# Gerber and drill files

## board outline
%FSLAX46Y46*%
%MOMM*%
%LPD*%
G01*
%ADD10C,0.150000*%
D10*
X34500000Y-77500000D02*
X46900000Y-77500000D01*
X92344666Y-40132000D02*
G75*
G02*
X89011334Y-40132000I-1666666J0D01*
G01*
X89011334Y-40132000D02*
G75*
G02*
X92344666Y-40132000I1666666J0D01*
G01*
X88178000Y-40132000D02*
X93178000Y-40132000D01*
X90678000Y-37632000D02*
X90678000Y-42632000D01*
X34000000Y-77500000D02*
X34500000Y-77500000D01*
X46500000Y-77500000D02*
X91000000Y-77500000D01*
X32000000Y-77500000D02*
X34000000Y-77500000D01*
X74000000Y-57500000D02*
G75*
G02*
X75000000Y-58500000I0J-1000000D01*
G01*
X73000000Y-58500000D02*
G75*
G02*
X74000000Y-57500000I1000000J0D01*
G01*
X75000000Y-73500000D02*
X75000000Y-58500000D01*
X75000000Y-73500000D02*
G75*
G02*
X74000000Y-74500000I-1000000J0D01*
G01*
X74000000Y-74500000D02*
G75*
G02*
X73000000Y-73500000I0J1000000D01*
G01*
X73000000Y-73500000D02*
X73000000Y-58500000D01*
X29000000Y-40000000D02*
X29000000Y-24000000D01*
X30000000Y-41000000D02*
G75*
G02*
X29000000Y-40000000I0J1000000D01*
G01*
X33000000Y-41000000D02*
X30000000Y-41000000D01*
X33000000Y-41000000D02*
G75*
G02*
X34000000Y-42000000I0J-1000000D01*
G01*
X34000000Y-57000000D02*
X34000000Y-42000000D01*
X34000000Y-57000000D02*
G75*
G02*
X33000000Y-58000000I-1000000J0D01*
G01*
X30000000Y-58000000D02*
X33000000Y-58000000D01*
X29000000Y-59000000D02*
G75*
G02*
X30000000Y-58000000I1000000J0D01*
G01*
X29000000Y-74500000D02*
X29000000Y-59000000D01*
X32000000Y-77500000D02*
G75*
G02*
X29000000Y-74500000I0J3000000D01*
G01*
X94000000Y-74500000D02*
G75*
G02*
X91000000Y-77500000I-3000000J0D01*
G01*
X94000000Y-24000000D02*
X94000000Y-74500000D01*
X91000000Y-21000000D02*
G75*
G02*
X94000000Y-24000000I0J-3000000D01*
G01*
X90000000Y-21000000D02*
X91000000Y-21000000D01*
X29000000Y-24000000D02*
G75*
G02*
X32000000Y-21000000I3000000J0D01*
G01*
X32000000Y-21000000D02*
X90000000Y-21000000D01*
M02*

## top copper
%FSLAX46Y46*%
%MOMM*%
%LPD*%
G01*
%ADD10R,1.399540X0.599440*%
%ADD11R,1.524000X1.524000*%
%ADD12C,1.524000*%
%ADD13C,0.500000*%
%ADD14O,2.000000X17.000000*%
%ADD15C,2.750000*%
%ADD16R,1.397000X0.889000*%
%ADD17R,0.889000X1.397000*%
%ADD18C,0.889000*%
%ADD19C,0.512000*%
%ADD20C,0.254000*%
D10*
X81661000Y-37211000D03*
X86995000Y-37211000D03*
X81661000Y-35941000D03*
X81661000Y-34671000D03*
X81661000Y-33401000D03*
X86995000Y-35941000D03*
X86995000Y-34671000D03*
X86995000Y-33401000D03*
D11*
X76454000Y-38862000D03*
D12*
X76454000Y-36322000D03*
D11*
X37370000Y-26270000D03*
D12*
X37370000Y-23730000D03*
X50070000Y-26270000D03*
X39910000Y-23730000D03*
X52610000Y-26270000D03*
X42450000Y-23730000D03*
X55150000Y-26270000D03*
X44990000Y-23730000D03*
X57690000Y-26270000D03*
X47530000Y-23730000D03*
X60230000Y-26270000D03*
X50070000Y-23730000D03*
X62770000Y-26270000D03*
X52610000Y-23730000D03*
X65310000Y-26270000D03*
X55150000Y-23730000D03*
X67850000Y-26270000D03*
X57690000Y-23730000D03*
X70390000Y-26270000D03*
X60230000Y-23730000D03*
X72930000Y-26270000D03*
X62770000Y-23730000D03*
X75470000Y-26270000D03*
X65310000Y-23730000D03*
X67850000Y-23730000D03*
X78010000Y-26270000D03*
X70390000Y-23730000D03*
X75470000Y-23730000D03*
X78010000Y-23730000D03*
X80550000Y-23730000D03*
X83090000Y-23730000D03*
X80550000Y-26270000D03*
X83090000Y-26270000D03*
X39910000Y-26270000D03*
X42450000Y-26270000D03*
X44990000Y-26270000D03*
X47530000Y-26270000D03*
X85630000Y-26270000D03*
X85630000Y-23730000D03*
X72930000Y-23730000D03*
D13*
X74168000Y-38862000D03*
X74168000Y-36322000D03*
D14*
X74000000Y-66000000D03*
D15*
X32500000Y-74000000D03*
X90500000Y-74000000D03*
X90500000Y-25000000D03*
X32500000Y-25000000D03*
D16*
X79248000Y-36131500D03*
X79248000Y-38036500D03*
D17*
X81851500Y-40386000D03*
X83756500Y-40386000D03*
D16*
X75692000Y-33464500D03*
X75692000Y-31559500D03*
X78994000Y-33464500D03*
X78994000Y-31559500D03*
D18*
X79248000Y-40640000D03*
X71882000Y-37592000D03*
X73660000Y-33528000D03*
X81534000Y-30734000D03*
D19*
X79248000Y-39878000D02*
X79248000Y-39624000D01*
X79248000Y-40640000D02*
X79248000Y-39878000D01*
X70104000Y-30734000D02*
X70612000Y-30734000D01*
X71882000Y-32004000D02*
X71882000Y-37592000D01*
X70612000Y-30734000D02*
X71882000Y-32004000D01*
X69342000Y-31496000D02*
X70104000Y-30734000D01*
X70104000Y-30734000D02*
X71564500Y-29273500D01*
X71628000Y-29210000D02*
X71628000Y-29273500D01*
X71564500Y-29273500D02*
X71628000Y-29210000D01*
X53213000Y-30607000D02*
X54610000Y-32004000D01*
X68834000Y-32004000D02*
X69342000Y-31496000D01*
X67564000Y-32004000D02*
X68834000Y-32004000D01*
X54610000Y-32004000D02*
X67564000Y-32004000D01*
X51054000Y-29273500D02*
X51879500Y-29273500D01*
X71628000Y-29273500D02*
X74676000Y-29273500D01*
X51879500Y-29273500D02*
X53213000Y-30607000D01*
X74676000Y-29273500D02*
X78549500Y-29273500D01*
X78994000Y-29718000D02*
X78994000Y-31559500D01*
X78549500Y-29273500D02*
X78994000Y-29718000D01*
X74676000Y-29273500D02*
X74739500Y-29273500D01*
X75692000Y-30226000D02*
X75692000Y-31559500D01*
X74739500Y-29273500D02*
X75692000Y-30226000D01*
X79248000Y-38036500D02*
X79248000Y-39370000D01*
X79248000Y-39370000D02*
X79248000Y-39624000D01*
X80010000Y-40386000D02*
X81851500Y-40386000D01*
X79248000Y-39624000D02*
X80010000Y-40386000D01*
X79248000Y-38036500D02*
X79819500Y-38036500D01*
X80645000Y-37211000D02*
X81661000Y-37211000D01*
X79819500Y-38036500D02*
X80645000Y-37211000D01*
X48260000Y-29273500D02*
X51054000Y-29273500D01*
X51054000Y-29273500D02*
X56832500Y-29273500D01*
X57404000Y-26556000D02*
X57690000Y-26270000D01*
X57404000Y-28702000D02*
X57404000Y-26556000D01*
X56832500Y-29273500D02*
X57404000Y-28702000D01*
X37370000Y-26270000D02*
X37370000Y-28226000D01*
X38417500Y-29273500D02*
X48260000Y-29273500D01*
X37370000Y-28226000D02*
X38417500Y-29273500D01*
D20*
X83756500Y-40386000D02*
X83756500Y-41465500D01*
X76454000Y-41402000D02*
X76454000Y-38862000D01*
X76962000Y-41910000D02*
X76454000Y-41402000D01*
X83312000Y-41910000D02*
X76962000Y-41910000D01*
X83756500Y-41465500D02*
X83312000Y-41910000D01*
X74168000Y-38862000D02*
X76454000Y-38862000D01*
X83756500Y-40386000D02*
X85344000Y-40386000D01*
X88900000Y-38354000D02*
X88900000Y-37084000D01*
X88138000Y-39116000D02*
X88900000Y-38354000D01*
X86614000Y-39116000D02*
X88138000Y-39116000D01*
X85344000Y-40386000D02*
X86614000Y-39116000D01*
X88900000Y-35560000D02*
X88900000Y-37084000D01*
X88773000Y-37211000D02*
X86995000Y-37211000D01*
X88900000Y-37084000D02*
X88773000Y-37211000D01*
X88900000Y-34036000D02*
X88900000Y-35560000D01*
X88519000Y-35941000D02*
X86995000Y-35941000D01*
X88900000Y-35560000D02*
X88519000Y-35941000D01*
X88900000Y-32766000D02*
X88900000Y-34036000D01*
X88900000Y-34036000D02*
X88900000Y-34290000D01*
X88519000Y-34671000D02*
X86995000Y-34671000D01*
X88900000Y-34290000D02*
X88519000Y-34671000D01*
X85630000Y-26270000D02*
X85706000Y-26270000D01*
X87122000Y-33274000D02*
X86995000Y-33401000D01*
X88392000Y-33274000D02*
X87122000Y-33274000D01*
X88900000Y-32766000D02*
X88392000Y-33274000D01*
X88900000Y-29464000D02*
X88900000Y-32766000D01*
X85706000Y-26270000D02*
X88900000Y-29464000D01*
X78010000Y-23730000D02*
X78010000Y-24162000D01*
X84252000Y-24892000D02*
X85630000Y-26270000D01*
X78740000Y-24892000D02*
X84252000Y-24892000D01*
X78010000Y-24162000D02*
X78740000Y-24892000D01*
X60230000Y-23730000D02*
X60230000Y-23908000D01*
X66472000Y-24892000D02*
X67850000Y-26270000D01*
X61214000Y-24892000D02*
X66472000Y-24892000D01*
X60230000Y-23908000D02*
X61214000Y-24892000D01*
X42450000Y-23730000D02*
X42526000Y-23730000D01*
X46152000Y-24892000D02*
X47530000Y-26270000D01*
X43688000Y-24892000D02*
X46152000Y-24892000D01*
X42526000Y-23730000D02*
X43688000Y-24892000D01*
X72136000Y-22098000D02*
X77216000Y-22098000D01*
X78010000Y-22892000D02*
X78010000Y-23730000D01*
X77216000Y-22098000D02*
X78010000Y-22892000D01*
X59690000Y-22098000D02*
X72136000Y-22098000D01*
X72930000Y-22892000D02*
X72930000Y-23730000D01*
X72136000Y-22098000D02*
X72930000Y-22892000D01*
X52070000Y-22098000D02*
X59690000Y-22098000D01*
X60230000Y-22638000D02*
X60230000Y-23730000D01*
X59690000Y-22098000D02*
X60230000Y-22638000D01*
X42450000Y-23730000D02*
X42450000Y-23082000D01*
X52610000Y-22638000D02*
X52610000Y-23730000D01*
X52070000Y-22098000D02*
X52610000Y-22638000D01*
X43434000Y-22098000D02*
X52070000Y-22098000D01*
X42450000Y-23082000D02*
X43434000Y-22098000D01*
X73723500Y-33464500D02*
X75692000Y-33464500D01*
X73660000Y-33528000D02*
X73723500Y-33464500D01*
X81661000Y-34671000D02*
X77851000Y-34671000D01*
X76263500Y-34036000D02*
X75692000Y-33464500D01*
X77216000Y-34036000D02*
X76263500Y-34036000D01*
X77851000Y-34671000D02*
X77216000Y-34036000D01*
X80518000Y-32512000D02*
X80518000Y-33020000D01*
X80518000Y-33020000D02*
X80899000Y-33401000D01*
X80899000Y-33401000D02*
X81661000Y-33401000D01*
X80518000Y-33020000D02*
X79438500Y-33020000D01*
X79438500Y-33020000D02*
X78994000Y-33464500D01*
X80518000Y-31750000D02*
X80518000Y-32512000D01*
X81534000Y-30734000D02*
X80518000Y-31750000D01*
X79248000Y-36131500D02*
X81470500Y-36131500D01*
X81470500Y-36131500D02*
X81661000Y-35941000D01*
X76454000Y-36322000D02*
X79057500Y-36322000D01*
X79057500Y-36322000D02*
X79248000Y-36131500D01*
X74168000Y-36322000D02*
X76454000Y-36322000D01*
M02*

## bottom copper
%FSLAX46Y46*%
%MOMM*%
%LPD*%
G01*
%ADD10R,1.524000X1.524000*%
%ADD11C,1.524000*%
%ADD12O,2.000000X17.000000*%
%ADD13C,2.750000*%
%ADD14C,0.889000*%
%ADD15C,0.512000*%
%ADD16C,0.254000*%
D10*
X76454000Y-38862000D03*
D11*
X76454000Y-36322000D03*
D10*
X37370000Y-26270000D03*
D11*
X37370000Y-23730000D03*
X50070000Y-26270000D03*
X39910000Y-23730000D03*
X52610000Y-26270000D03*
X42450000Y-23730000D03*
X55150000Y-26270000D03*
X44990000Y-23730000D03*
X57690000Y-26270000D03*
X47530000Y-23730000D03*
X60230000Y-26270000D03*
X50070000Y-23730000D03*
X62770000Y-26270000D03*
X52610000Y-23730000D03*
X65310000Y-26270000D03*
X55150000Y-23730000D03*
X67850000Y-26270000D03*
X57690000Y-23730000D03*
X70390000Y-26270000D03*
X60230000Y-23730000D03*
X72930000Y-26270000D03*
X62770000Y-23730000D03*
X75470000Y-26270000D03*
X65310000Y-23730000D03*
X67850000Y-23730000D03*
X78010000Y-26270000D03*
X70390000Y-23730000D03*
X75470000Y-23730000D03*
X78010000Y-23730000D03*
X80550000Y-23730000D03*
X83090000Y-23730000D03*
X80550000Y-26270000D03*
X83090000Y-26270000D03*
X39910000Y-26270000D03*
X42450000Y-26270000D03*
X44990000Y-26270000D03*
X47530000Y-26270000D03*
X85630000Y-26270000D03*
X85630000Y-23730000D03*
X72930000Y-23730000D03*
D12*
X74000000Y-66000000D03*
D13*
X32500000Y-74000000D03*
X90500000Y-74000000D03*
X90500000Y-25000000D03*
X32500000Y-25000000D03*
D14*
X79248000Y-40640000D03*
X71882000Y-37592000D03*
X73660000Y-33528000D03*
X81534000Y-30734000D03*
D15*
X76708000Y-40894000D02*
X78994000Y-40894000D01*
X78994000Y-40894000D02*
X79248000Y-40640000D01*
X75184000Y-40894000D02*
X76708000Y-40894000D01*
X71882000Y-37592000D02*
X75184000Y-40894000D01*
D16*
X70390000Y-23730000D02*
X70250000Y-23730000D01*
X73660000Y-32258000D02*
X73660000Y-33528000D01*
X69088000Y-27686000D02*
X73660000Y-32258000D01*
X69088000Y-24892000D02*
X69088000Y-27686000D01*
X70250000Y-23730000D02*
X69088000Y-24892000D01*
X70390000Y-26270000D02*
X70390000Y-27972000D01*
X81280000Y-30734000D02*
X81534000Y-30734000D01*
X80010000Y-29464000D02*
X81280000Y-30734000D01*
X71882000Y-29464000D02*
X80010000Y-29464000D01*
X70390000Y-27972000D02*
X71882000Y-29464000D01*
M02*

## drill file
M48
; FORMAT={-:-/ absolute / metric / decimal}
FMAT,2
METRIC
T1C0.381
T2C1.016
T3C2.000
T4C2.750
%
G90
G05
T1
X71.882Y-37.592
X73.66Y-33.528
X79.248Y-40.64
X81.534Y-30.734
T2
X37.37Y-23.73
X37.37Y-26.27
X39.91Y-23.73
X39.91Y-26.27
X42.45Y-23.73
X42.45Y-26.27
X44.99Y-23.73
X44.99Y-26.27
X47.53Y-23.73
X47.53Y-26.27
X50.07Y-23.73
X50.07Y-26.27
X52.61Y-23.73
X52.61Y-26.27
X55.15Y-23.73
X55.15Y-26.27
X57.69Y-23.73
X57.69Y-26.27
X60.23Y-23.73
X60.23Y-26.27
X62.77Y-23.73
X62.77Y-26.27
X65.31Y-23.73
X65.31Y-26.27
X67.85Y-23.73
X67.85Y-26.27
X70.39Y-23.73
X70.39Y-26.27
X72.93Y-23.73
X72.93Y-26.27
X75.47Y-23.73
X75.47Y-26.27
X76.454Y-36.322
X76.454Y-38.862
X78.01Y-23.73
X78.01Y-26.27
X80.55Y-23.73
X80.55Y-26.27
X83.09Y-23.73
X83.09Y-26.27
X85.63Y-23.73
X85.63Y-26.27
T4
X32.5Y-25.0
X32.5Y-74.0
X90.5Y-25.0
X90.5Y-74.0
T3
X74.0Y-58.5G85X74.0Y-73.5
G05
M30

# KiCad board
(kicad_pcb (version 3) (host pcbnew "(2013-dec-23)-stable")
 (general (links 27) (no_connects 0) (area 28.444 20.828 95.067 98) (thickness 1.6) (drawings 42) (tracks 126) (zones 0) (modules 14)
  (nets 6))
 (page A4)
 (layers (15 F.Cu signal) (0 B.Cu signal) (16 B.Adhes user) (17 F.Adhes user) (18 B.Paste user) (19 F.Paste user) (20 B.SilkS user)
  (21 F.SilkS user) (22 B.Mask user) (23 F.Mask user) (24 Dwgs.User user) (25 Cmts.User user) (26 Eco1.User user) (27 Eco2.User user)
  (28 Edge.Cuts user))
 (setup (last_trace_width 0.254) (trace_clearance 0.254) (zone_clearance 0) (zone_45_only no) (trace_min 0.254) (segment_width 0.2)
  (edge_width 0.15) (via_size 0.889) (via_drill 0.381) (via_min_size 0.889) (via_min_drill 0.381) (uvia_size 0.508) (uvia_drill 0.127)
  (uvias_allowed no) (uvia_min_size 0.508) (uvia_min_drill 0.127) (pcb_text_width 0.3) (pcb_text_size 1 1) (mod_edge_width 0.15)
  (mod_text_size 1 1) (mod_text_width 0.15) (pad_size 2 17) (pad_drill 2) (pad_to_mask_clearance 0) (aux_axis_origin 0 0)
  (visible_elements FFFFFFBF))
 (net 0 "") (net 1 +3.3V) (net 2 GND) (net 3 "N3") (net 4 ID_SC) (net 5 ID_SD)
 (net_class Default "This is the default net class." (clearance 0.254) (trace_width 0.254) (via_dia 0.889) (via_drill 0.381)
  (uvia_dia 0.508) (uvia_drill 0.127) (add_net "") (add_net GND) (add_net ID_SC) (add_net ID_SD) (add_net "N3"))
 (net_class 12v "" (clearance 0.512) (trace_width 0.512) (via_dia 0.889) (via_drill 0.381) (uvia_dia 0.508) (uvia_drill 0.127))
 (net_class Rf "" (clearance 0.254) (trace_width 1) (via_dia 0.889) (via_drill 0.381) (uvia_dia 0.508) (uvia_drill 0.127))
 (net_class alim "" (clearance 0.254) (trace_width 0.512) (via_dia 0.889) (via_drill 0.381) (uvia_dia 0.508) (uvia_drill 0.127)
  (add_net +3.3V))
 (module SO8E (layer F.Cu) (at 84.328 35.306 90)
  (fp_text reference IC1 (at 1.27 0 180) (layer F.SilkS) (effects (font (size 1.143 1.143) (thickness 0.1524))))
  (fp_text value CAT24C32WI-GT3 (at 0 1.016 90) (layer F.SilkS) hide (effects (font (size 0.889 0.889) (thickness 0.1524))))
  (pad 8 smd rect (at -1.905 -2.667 90) (size 0.59944 1.39954) (layers F.Cu F.Paste F.Mask) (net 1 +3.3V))
  (pad 1 smd rect (at -1.905 2.667 90) (size 0.59944 1.39954) (layers F.Cu F.Paste F.Mask) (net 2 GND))
  (pad 7 smd rect (at -0.635 -2.667 90) (size 0.59944 1.39954) (layers F.Cu F.Paste F.Mask) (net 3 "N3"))
  (pad 6 smd rect (at 0.635 -2.667 90) (size 0.59944 1.39954) (layers F.Cu F.Paste F.Mask) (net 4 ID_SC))
  (pad 5 smd rect (at 1.905 -2.667 90) (size 0.59944 1.39954) (layers F.Cu F.Paste F.Mask) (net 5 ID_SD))
  (pad 2 smd rect (at -0.635 2.667 90) (size 0.59944 1.39954) (layers F.Cu F.Paste F.Mask) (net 2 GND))
  (pad 3 smd rect (at 0.635 2.667 90) (size 0.59944 1.39954) (layers F.Cu F.Paste F.Mask) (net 2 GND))
  (pad 4 smd rect (at 1.905 2.667 90) (size 0.59944 1.39954) (layers F.Cu F.Paste F.Mask) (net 2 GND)))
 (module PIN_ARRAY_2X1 (layer F.Cu) (at 76.454 37.592 90)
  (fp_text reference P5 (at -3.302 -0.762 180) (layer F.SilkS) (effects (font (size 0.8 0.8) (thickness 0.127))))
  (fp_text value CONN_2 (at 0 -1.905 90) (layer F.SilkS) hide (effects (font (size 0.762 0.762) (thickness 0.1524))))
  (pad 1 thru_hole rect (at -1.27 0 90) (size 1.524 1.524) (drill 1.016) (layers *.Cu *.Mask F.SilkS) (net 2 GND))
  (pad 2 thru_hole circle (at 1.27 0 90) (size 1.524 1.524) (drill 1.016) (layers *.Cu *.Mask F.SilkS) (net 3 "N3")))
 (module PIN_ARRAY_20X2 (layer F.Cu) (at 61.5 25)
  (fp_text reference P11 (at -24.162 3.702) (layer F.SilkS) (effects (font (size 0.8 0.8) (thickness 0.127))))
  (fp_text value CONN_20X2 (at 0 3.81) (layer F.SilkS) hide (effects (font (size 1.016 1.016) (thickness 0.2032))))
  (pad 1 thru_hole rect (at -24.13 1.27) (size 1.524 1.524) (drill 1.016) (layers *.Cu *.Mask F.SilkS) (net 1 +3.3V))
  (pad 2 thru_hole circle (at -24.13 -1.27) (size 1.524 1.524) (drill 1.016) (layers *.Cu *.Mask F.SilkS))
  (pad 11 thru_hole circle (at -11.43 1.27) (size 1.524 1.524) (drill 1.016) (layers *.Cu *.Mask F.SilkS))
  (pad 4 thru_hole circle (at -21.59 -1.27) (size 1.524 1.524) (drill 1.016) (layers *.Cu *.Mask F.SilkS))
  (pad 13 thru_hole circle (at -8.89 1.27) (size 1.524 1.524) (drill 1.016) (layers *.Cu *.Mask F.SilkS))
  (pad 6 thru_hole circle (at -19.05 -1.27) (size 1.524 1.524) (drill 1.016) (layers *.Cu *.Mask F.SilkS) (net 2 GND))
  (pad 15 thru_hole circle (at -6.35 1.27) (size 1.524 1.524) (drill 1.016) (layers *.Cu *.Mask F.SilkS))
  (pad 8 thru_hole circle (at -16.51 -1.27) (size 1.524 1.524) (drill 1.016) (layers *.Cu *.Mask F.SilkS))
  (pad 17 thru_hole circle (at -3.81 1.27) (size 1.524 1.524) (drill 1.016) (layers *.Cu *.Mask F.SilkS) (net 1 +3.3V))
  (pad 10 thru_hole circle (at -13.97 -1.27) (size 1.524 1.524) (drill 1.016) (layers *.Cu *.Mask F.SilkS))
  (pad 19 thru_hole circle (at -1.27 1.27) (size 1.524 1.524) (drill 1.016) (layers *.Cu *.Mask F.SilkS))
  (pad 12 thru_hole circle (at -11.43 -1.27) (size 1.524 1.524) (drill 1.016) (layers *.Cu *.Mask F.SilkS))
  (pad 21 thru_hole circle (at 1.27 1.27) (size 1.524 1.524) (drill 1.016) (layers *.Cu *.Mask F.SilkS))
  (pad 14 thru_hole circle (at -8.89 -1.27) (size 1.524 1.524) (drill 1.016) (layers *.Cu *.Mask F.SilkS) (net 2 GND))
  (pad 23 thru_hole circle (at 3.81 1.27) (size 1.524 1.524) (drill 1.016) (layers *.Cu *.Mask F.SilkS))
  (pad 16 thru_hole circle (at -6.35 -1.27) (size 1.524 1.524) (drill 1.016) (layers *.Cu *.Mask F.SilkS))
  (pad 25 thru_hole circle (at 6.35 1.27) (size 1.524 1.524) (drill 1.016) (layers *.Cu *.Mask F.SilkS) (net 2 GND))
  (pad 18 thru_hole circle (at -3.81 -1.27) (size 1.524 1.524) (drill 1.016) (layers *.Cu *.Mask F.SilkS))
  (pad 27 thru_hole circle (at 8.89 1.27) (size 1.524 1.524) (drill 1.016) (layers *.Cu *.Mask F.SilkS) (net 5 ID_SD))
  (pad 20 thru_hole circle (at -1.27 -1.27) (size 1.524 1.524) (drill 1.016) (layers *.Cu *.Mask F.SilkS) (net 2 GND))
  (pad 29 thru_hole circle (at 11.43 1.27) (size 1.524 1.524) (drill 1.016) (layers *.Cu *.Mask F.SilkS))
  (pad 22 thru_hole circle (at 1.27 -1.27) (size 1.524 1.524) (drill 1.016) (layers *.Cu *.Mask F.SilkS))
  (pad 31 thru_hole circle (at 13.97 1.27) (size 1.524 1.524) (drill 1.016) (layers *.Cu *.Mask F.SilkS))
  (pad 24 thru_hole circle (at 3.81 -1.27) (size 1.524 1.524) (drill 1.016) (layers *.Cu *.Mask F.SilkS))
  (pad 26 thru_hole circle (at 6.35 -1.27) (size 1.524 1.524) (drill 1.016) (layers *.Cu *.Mask F.SilkS))
  (pad 33 thru_hole circle (at 16.51 1.27) (size 1.524 1.524) (drill 1.016) (layers *.Cu *.Mask F.SilkS))
  (pad 28 thru_hole circle (at 8.89 -1.27) (size 1.524 1.524) (drill 1.016) (layers *.Cu *.Mask F.SilkS) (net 4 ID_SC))
  (pad 32 thru_hole circle (at 13.97 -1.27) (size 1.524 1.524) (drill 1.016) (layers *.Cu *.Mask F.SilkS))
  (pad 34 thru_hole circle (at 16.51 -1.27) (size 1.524 1.524) (drill 1.016) (layers *.Cu *.Mask F.SilkS) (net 2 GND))
  (pad 36 thru_hole circle (at 19.05 -1.27) (size 1.524 1.524) (drill 1.016) (layers *.Cu *.Mask F.SilkS))
  (pad 38 thru_hole circle (at 21.59 -1.27) (size 1.524 1.524) (drill 1.016) (layers *.Cu *.Mask F.SilkS))
  (pad 35 thru_hole circle (at 19.05 1.27) (size 1.524 1.524) (drill 1.016) (layers *.Cu *.Mask F.SilkS))
  (pad 37 thru_hole circle (at 21.59 1.27) (size 1.524 1.524) (drill 1.016) (layers *.Cu *.Mask F.SilkS))
  (pad 3 thru_hole circle (at -21.59 1.27) (size 1.524 1.524) (drill 1.016) (layers *.Cu *.Mask F.SilkS))
  (pad 5 thru_hole circle (at -19.05 1.27) (size 1.524 1.524) (drill 1.016) (layers *.Cu *.Mask F.SilkS))
  (pad 7 thru_hole circle (at -16.51 1.27) (size 1.524 1.524) (drill 1.016) (layers *.Cu *.Mask F.SilkS))
  (pad 9 thru_hole circle (at -13.97 1.27) (size 1.524 1.524) (drill 1.016) (layers *.Cu *.Mask F.SilkS) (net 2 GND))
  (pad 39 thru_hole circle (at 24.13 1.27) (size 1.524 1.524) (drill 1.016) (layers *.Cu *.Mask F.SilkS) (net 2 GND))
  (pad 40 thru_hole circle (at 24.13 -1.27) (size 1.524 1.524) (drill 1.016) (layers *.Cu *.Mask F.SilkS))
  (pad 30 thru_hole circle (at 11.43 -1.27) (size 1.524 1.524) (drill 1.016) (layers *.Cu *.Mask F.SilkS) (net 2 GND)))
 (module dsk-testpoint (layer F.Cu) (at 74.168 38.862)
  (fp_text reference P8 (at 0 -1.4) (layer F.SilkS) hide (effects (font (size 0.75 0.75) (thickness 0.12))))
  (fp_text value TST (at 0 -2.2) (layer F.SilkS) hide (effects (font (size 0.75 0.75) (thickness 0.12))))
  (pad 1 smd circle (at 0 0) (size 0.5 0.5) (layers F.Cu F.Paste F.Mask) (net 2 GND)))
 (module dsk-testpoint (layer F.Cu) (at 74.168 36.322)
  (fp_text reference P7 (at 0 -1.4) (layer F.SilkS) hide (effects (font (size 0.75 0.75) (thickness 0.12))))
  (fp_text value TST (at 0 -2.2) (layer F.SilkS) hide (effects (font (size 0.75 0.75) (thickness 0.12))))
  (pad 1 smd circle (at 0 0) (size 0.5 0.5) (layers F.Cu F.Paste F.Mask) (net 3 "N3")))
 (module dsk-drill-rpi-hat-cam (layer F.Cu) (at 74 66)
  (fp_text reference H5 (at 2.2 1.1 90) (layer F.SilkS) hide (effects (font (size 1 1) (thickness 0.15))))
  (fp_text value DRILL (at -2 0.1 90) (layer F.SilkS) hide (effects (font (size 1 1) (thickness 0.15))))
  (pad 1 thru_hole oval (at 0 0) (size 2 17) (drill oval 2 17) (layers *.Cu F.SilkS) (solder_mask_margin 0.254) (clearance 0.254)))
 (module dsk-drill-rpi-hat (layer F.Cu) (at 32.5 74)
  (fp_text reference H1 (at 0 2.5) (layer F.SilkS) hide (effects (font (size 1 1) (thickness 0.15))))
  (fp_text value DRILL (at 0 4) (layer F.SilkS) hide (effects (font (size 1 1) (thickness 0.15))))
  (pad 1 thru_hole circle (at 0 0) (size 2.75 2.75) (drill 2.75) (layers *.Cu) (solder_mask_margin 1.725) (clearance 1.725) (zone_connect 0)))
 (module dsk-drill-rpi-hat (layer F.Cu) (at 90.5 74)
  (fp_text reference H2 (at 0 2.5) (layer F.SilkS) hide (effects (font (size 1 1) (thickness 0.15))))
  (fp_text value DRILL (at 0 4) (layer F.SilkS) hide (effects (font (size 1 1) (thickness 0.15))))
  (pad 1 thru_hole circle (at 0 0) (size 2.75 2.75) (drill 2.75) (layers *.Cu) (solder_mask_margin 1.725) (clearance 1.725) (zone_connect 0)))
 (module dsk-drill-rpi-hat (layer F.Cu) (at 90.5 25)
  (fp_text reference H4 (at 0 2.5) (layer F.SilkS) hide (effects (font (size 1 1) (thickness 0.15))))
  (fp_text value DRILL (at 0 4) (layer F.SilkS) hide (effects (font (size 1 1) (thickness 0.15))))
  (pad 1 thru_hole circle (at 0 0) (size 2.75 2.75) (drill 2.75) (layers *.Cu) (solder_mask_margin 1.725) (clearance 1.725) (zone_connect 0)))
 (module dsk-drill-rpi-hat (layer F.Cu) (at 32.5 25)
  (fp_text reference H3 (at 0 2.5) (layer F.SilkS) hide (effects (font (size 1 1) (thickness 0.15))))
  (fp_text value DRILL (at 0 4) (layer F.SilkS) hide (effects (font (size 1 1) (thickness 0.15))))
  (pad 1 thru_hole circle (at 0 0) (size 2.75 2.75) (drill 2.75) (layers *.Cu) (solder_mask_margin 1.725) (clearance 1.725) (zone_connect 0)))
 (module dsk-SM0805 (layer F.Cu) (at 79.248 37.084 270)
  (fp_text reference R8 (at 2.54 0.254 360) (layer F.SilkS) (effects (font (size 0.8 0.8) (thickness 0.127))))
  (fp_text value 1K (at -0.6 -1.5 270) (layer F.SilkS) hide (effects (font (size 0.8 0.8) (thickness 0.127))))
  (pad 1 smd rect (at -0.9525 0 270) (size 0.889 1.397) (layers F.Cu F.Paste F.Mask) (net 3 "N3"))
  (pad 2 smd rect (at 0.9525 0 270) (size 0.889 1.397) (layers F.Cu F.Paste F.Mask) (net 1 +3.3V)))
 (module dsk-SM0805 (layer F.Cu) (at 82.804 40.386)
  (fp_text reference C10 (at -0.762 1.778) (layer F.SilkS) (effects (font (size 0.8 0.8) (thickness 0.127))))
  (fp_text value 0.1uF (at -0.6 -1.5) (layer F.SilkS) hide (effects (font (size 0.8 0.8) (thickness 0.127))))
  (pad 1 smd rect (at -0.9525 0) (size 0.889 1.397) (layers F.Cu F.Paste F.Mask) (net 1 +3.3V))
  (pad 2 smd rect (at 0.9525 0) (size 0.889 1.397) (layers F.Cu F.Paste F.Mask) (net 2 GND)))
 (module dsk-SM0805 (layer F.Cu) (at 75.692 32.512 90)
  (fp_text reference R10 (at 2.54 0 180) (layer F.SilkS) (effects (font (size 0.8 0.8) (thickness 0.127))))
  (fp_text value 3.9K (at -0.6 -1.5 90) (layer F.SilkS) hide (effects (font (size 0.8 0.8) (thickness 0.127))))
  (pad 1 smd rect (at -0.9525 0 90) (size 0.889 1.397) (layers F.Cu F.Paste F.Mask) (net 4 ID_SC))
  (pad 2 smd rect (at 0.9525 0 90) (size 0.889 1.397) (layers F.Cu F.Paste F.Mask) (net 1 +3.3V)))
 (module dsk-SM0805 (layer F.Cu) (at 78.994 32.512 90)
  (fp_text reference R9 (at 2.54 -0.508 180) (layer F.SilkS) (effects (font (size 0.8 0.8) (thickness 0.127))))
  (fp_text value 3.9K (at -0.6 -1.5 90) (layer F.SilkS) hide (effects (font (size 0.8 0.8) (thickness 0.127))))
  (pad 1 smd rect (at -0.9525 0 90) (size 0.889 1.397) (layers F.Cu F.Paste F.Mask) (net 5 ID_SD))
  (pad 2 smd rect (at 0.9525 0 90) (size 0.889 1.397) (layers F.Cu F.Paste F.Mask) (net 1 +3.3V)))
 (gr_line (start 34.5 77.5) (end 46.9 77.5) (angle 90) (layer Edge.Cuts) (width 0.15))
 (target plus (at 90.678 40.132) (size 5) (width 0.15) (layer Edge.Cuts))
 (gr_line (start 34 77.5) (end 34.5 77.5) (angle 90) (layer Edge.Cuts) (width 0.15))
 (gr_line (start 46.5 77.5) (end 91 77.5) (angle 90) (layer Edge.Cuts) (width 0.15))
 (gr_line (start 32 77.5) (end 34 77.5) (angle 90) (layer Edge.Cuts) (width 0.15))
 (gr_arc (start 74 58.5) (end 74 57.5) (angle 90) (layer Edge.Cuts) (width 0.15))
 (gr_arc (start 74 58.5) (end 73 58.5) (angle 90) (layer Edge.Cuts) (width 0.15))
 (gr_line (start 75 73.5) (end 75 58.5) (angle 90) (layer Edge.Cuts) (width 0.15))
 (gr_arc (start 74 73.5) (end 75 73.5) (angle 90) (layer Edge.Cuts) (width 0.15))
 (gr_arc (start 74 73.5) (end 74 74.5) (angle 90) (layer Edge.Cuts) (width 0.15))
 (gr_line (start 73 73.5) (end 73 58.5) (angle 90) (layer Edge.Cuts) (width 0.15))
 (gr_line (start 29 40) (end 29 24) (angle 90) (layer Edge.Cuts) (width 0.15))
 (gr_arc (start 30 40) (end 30 41) (angle 90) (layer Edge.Cuts) (width 0.15))
 (gr_line (start 33 41) (end 30 41) (angle 90) (layer Edge.Cuts) (width 0.15))
 (gr_arc (start 33 42) (end 33 41) (angle 90) (layer Edge.Cuts) (width 0.15))
 (gr_line (start 34 57) (end 34 42) (angle 90) (layer Edge.Cuts) (width 0.15))
 (gr_arc (start 33 57) (end 34 57) (angle 90) (layer Edge.Cuts) (width 0.15))
 (gr_line (start 30 58) (end 33 58) (angle 90) (layer Edge.Cuts) (width 0.15))
 (gr_arc (start 30 59) (end 29 59) (angle 90) (layer Edge.Cuts) (width 0.15))
 (gr_line (start 29 74.5) (end 29 59) (angle 90) (layer Edge.Cuts) (width 0.15))
 (gr_arc (start 32 74.5) (end 32 77.5) (angle 90) (layer Edge.Cuts) (width 0.15))
 (gr_arc (start 91 74.5) (end 94 74.5) (angle 90) (layer Edge.Cuts) (width 0.15))
 (gr_line (start 94 24) (end 94 74.5) (angle 90) (layer Edge.Cuts) (width 0.15))
 (gr_arc (start 91 24) (end 91 21) (angle 90) (layer Edge.Cuts) (width 0.15))
 (gr_line (start 90 21) (end 91 21) (angle 90) (layer Edge.Cuts) (width 0.15))
 (gr_arc (start 32 24) (end 29 24) (angle 90) (layer Edge.Cuts) (width 0.15))
 (gr_line (start 32 21) (end 90 21) (angle 90) (layer Edge.Cuts) (width 0.15))
 (segment (start 76.708 40.894) (end 78.994 40.894) (width 0.512) (layer B.Cu) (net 1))
 (segment (start 79.248 39.878) (end 79.248 39.624) (width 0.512) (layer F.Cu) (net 1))
 (segment (start 79.248 40.64) (end 79.248 39.878) (width 0.512) (layer F.Cu) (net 1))
 (via (at 79.248 40.64) (size 0.889) (layers F.Cu B.Cu) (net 1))
 (segment (start 78.994 40.894) (end 79.248 40.64) (width 0.512) (layer B.Cu) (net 1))
 (segment (start 70.104 30.734) (end 70.612 30.734) (width 0.512) (layer F.Cu) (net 1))
 (segment (start 75.184 40.894) (end 76.708 40.894) (width 0.512) (layer B.Cu) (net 1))
 (segment (start 71.882 37.592) (end 75.184 40.894) (width 0.512) (layer B.Cu) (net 1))
 (via (at 71.882 37.592) (size 0.889) (layers F.Cu B.Cu) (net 1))
 (segment (start 71.882 32.004) (end 71.882 37.592) (width 0.512) (layer F.Cu) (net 1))
 (segment (start 70.612 30.734) (end 71.882 32.004) (width 0.512) (layer F.Cu) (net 1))
 (segment (start 69.342 31.496) (end 70.104 30.734) (width 0.512) (layer F.Cu) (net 1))
 (segment (start 70.104 30.734) (end 71.5645 29.2735) (width 0.512) (layer F.Cu) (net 1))
 (segment (start 71.628 29.21) (end 71.628 29.2735) (width 0.512) (layer F.Cu) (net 1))
 (segment (start 71.5645 29.2735) (end 71.628 29.21) (width 0.512) (layer F.Cu) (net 1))
 (segment (start 53.213 30.607) (end 54.61 32.004) (width 0.512) (layer F.Cu) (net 1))
 (segment (start 68.834 32.004) (end 69.342 31.496) (width 0.512) (layer F.Cu) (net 1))
 (segment (start 67.564 32.004) (end 68.834 32.004) (width 0.512) (layer F.Cu) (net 1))
 (segment (start 54.61 32.004) (end 67.564 32.004) (width 0.512) (layer F.Cu) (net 1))
 (segment (start 51.054 29.2735) (end 51.8795 29.2735) (width 0.512) (layer F.Cu) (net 1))
 (segment (start 71.628 29.2735) (end 74.676 29.2735) (width 0.512) (layer F.Cu) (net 1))
 (segment (start 51.8795 29.2735) (end 53.213 30.607) (width 0.512) (layer F.Cu) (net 1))
 (segment (start 74.676 29.2735) (end 78.5495 29.2735) (width 0.512) (layer F.Cu) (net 1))
 (segment (start 78.994 29.718) (end 78.994 31.5595) (width 0.512) (layer F.Cu) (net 1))
 (segment (start 78.5495 29.2735) (end 78.994 29.718) (width 0.512) (layer F.Cu) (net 1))
 (segment (start 74.676 29.2735) (end 74.7395 29.2735) (width 0.512) (layer F.Cu) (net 1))
 (segment (start 75.692 30.226) (end 75.692 31.5595) (width 0.512) (layer F.Cu) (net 1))
 (segment (start 74.7395 29.2735) (end 75.692 30.226) (width 0.512) (layer F.Cu) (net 1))
 (segment (start 79.248 38.0365) (end 79.248 39.37) (width 0.512) (layer F.Cu) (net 1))
 (segment (start 79.248 39.37) (end 79.248 39.624) (width 0.512) (layer F.Cu) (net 1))
 (segment (start 80.01 40.386) (end 81.8515 40.386) (width 0.512) (layer F.Cu) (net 1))
 (segment (start 79.248 39.624) (end 80.01 40.386) (width 0.512) (layer F.Cu) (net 1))
 (segment (start 79.248 38.0365) (end 79.8195 38.0365) (width 0.512) (layer F.Cu) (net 1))
 (segment (start 80.645 37.211) (end 81.661 37.211) (width 0.512) (layer F.Cu) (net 1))
 (segment (start 79.8195 38.0365) (end 80.645 37.211) (width 0.512) (layer F.Cu) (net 1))
 (segment (start 48.26 29.2735) (end 51.054 29.2735) (width 0.512) (layer F.Cu) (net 1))
 (segment (start 51.054 29.2735) (end 56.8325 29.2735) (width 0.512) (layer F.Cu) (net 1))
 (segment (start 57.404 26.556) (end 57.69 26.27) (width 0.512) (layer F.Cu) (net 1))
 (segment (start 57.404 28.702) (end 57.404 26.556) (width 0.512) (layer F.Cu) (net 1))
 (segment (start 56.8325 29.2735) (end 57.404 28.702) (width 0.512) (layer F.Cu) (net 1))
 (segment (start 37.37 26.27) (end 37.37 28.226) (width 0.512) (layer F.Cu) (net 1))
 (segment (start 38.4175 29.2735) (end 48.26 29.2735) (width 0.512) (layer F.Cu) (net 1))
 (segment (start 37.37 28.226) (end 38.4175 29.2735) (width 0.512) (layer F.Cu) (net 1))
 (segment (start 83.7565 40.386) (end 83.7565 41.4655) (width 0.254) (layer F.Cu) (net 2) (status 400000))
 (segment (start 76.454 41.402) (end 76.454 38.862) (width 0.254) (layer F.Cu) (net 2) (status 800000))
 (segment (start 76.962 41.91) (end 76.454 41.402) (width 0.254) (layer F.Cu) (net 2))
 (segment (start 83.312 41.91) (end 76.962 41.91) (width 0.254) (layer F.Cu) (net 2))
 (segment (start 83.7565 41.4655) (end 83.312 41.91) (width 0.254) (layer F.Cu) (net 2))
 (segment (start 74.168 38.862) (end 76.454 38.862) (width 0.254) (layer F.Cu) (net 2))
 (segment (start 83.7565 40.386) (end 85.344 40.386) (width 0.254) (layer F.Cu) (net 2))
 (segment (start 88.9 38.354) (end 88.9 37.084) (width 0.254) (layer F.Cu) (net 2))
 (segment (start 88.138 39.116) (end 88.9 38.354) (width 0.254) (layer F.Cu) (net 2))
 (segment (start 86.614 39.116) (end 88.138 39.116) (width 0.254) (layer F.Cu) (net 2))
 (segment (start 85.344 40.386) (end 86.614 39.116) (width 0.254) (layer F.Cu) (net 2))
 (segment (start 88.9 35.56) (end 88.9 37.084) (width 0.254) (layer F.Cu) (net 2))
 (segment (start 88.773 37.211) (end 86.995 37.211) (width 0.254) (layer F.Cu) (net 2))
 (segment (start 88.9 37.084) (end 88.773 37.211) (width 0.254) (layer F.Cu) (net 2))
 (segment (start 88.9 34.036) (end 88.9 35.56) (width 0.254) (layer F.Cu) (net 2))
 (segment (start 88.519 35.941) (end 86.995 35.941) (width 0.254) (layer F.Cu) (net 2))
 (segment (start 88.9 35.56) (end 88.519 35.941) (width 0.254) (layer F.Cu) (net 2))
 (segment (start 88.9 32.766) (end 88.9 34.036) (width 0.254) (layer F.Cu) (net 2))
 (segment (start 88.9 34.036) (end 88.9 34.29) (width 0.254) (layer F.Cu) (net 2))
 (segment (start 88.519 34.671) (end 86.995 34.671) (width 0.254) (layer F.Cu) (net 2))
 (segment (start 88.9 34.29) (end 88.519 34.671) (width 0.254) (layer F.Cu) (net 2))
 (segment (start 85.63 26.27) (end 85.706 26.27) (width 0.254) (layer F.Cu) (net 2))
 (segment (start 87.122 33.274) (end 86.995 33.401) (width 0.254) (layer F.Cu) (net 2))
 (segment (start 88.392 33.274) (end 87.122 33.274) (width 0.254) (layer F.Cu) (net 2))
 (segment (start 88.9 32.766) (end 88.392 33.274) (width 0.254) (layer F.Cu) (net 2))
 (segment (start 88.9 29.464) (end 88.9 32.766) (width 0.254) (layer F.Cu) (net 2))
 (segment (start 85.706 26.27) (end 88.9 29.464) (width 0.254) (layer F.Cu) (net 2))
 (segment (start 78.01 23.73) (end 78.01 24.162) (width 0.254) (layer F.Cu) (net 2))
 (segment (start 84.252 24.892) (end 85.63 26.27) (width 0.254) (layer F.Cu) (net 2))
 (segment (start 78.74 24.892) (end 84.252 24.892) (width 0.254) (layer F.Cu) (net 2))
 (segment (start 78.01 24.162) (end 78.74 24.892) (width 0.254) (layer F.Cu) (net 2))
 (segment (start 60.23 23.73) (end 60.23 23.908) (width 0.254) (layer F.Cu) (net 2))
 (segment (start 66.472 24.892) (end 67.85 26.27) (width 0.254) (layer F.Cu) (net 2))
 (segment (start 61.214 24.892) (end 66.472 24.892) (width 0.254) (layer F.Cu) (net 2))
 (segment (start 60.23 23.908) (end 61.214 24.892) (width 0.254) (layer F.Cu) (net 2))
 (segment (start 42.45 23.73) (end 42.526 23.73) (width 0.254) (layer F.Cu) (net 2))
 (segment (start 46.152 24.892) (end 47.53 26.27) (width 0.254) (layer F.Cu) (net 2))
 (segment (start 43.688 24.892) (end 46.152 24.892) (width 0.254) (layer F.Cu) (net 2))
 (segment (start 42.526 23.73) (end 43.688 24.892) (width 0.254) (layer F.Cu) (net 2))
 (segment (start 72.136 22.098) (end 77.216 22.098) (width 0.254) (layer F.Cu) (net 2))
 (segment (start 78.01 22.892) (end 78.01 23.73) (width 0.254) (layer F.Cu) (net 2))
 (segment (start 77.216 22.098) (end 78.01 22.892) (width 0.254) (layer F.Cu) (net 2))
 (segment (start 59.69 22.098) (end 72.136 22.098) (width 0.254) (layer F.Cu) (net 2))
 (segment (start 72.93 22.892) (end 72.93 23.73) (width 0.254) (layer F.Cu) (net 2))
 (segment (start 72.136 22.098) (end 72.93 22.892) (width 0.254) (layer F.Cu) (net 2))
 (segment (start 52.07 22.098) (end 59.69 22.098) (width 0.254) (layer F.Cu) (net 2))
 (segment (start 60.23 22.638) (end 60.23 23.73) (width 0.254) (layer F.Cu) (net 2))
 (segment (start 59.69 22.098) (end 60.23 22.638) (width 0.254) (layer F.Cu) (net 2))
 (segment (start 42.45 23.73) (end 42.45 23.082) (width 0.254) (layer F.Cu) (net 2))
 (segment (start 52.61 22.638) (end 52.61 23.73) (width 0.254) (layer F.Cu) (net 2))
 (segment (start 52.07 22.098) (end 52.61 22.638) (width 0.254) (layer F.Cu) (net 2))
 (segment (start 43.434 22.098) (end 52.07 22.098) (width 0.254) (layer F.Cu) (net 2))
 (segment (start 42.45 23.082) (end 43.434 22.098) (width 0.254) (layer F.Cu) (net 2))
 (segment (start 70.39 23.73) (end 70.25 23.73) (width 0.254) (layer B.Cu) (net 4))
 (segment (start 73.7235 33.4645) (end 75.692 33.4645) (width 0.254) (layer F.Cu) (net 4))
 (segment (start 73.66 33.528) (end 73.7235 33.4645) (width 0.254) (layer F.Cu) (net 4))
 (via (at 73.66 33.528) (size 0.889) (layers F.Cu B.Cu) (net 4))
 (segment (start 73.66 32.258) (end 73.66 33.528) (width 0.254) (layer B.Cu) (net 4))
 (segment (start 69.088 27.686) (end 73.66 32.258) (width 0.254) (layer B.Cu) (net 4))
 (segment (start 69.088 24.892) (end 69.088 27.686) (width 0.254) (layer B.Cu) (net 4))
 (segment (start 70.25 23.73) (end 69.088 24.892) (width 0.254) (layer B.Cu) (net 4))
 (segment (start 81.661 34.671) (end 77.851 34.671) (width 0.254) (layer F.Cu) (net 4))
 (segment (start 76.2635 34.036) (end 75.692 33.4645) (width 0.254) (layer F.Cu) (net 4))
 (segment (start 77.216 34.036) (end 76.2635 34.036) (width 0.254) (layer F.Cu) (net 4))
 (segment (start 77.851 34.671) (end 77.216 34.036) (width 0.254) (layer F.Cu) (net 4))
 (segment (start 80.518 32.512) (end 80.518 33.02) (width 0.254) (layer F.Cu) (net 5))
 (segment (start 80.518 33.02) (end 80.899 33.401) (width 0.254) (layer F.Cu) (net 5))
 (segment (start 80.899 33.401) (end 81.661 33.401) (width 0.254) (layer F.Cu) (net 5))
 (segment (start 80.518 33.02) (end 79.4385 33.02) (width 0.254) (layer F.Cu) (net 5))
 (segment (start 79.4385 33.02) (end 78.994 33.4645) (width 0.254) (layer F.Cu) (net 5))
 (segment (start 70.39 26.27) (end 70.39 27.972) (width 0.254) (layer B.Cu) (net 5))
 (segment (start 80.518 31.75) (end 80.518 32.512) (width 0.254) (layer F.Cu) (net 5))
 (segment (start 81.534 30.734) (end 80.518 31.75) (width 0.254) (layer F.Cu) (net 5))
 (via (at 81.534 30.734) (size 0.889) (layers F.Cu B.Cu) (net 5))
 (segment (start 81.28 30.734) (end 81.534 30.734) (width 0.254) (layer B.Cu) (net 5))
 (segment (start 80.01 29.464) (end 81.28 30.734) (width 0.254) (layer B.Cu) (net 5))
 (segment (start 71.882 29.464) (end 80.01 29.464) (width 0.254) (layer B.Cu) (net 5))
 (segment (start 70.39 27.972) (end 71.882 29.464) (width 0.254) (layer B.Cu) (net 5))
 (segment (start 79.248 36.1315) (end 81.4705 36.1315) (width 0.254) (layer F.Cu) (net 3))
 (segment (start 81.4705 36.1315) (end 81.661 35.941) (width 0.254) (layer F.Cu) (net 3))
 (segment (start 76.454 36.322) (end 79.0575 36.322) (width 0.254) (layer F.Cu) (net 3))
 (segment (start 79.0575 36.322) (end 79.248 36.1315) (width 0.254) (layer F.Cu) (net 3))
 (segment (start 74.168 36.322) (end 76.454 36.322) (width 0.254) (layer F.Cu) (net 3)))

